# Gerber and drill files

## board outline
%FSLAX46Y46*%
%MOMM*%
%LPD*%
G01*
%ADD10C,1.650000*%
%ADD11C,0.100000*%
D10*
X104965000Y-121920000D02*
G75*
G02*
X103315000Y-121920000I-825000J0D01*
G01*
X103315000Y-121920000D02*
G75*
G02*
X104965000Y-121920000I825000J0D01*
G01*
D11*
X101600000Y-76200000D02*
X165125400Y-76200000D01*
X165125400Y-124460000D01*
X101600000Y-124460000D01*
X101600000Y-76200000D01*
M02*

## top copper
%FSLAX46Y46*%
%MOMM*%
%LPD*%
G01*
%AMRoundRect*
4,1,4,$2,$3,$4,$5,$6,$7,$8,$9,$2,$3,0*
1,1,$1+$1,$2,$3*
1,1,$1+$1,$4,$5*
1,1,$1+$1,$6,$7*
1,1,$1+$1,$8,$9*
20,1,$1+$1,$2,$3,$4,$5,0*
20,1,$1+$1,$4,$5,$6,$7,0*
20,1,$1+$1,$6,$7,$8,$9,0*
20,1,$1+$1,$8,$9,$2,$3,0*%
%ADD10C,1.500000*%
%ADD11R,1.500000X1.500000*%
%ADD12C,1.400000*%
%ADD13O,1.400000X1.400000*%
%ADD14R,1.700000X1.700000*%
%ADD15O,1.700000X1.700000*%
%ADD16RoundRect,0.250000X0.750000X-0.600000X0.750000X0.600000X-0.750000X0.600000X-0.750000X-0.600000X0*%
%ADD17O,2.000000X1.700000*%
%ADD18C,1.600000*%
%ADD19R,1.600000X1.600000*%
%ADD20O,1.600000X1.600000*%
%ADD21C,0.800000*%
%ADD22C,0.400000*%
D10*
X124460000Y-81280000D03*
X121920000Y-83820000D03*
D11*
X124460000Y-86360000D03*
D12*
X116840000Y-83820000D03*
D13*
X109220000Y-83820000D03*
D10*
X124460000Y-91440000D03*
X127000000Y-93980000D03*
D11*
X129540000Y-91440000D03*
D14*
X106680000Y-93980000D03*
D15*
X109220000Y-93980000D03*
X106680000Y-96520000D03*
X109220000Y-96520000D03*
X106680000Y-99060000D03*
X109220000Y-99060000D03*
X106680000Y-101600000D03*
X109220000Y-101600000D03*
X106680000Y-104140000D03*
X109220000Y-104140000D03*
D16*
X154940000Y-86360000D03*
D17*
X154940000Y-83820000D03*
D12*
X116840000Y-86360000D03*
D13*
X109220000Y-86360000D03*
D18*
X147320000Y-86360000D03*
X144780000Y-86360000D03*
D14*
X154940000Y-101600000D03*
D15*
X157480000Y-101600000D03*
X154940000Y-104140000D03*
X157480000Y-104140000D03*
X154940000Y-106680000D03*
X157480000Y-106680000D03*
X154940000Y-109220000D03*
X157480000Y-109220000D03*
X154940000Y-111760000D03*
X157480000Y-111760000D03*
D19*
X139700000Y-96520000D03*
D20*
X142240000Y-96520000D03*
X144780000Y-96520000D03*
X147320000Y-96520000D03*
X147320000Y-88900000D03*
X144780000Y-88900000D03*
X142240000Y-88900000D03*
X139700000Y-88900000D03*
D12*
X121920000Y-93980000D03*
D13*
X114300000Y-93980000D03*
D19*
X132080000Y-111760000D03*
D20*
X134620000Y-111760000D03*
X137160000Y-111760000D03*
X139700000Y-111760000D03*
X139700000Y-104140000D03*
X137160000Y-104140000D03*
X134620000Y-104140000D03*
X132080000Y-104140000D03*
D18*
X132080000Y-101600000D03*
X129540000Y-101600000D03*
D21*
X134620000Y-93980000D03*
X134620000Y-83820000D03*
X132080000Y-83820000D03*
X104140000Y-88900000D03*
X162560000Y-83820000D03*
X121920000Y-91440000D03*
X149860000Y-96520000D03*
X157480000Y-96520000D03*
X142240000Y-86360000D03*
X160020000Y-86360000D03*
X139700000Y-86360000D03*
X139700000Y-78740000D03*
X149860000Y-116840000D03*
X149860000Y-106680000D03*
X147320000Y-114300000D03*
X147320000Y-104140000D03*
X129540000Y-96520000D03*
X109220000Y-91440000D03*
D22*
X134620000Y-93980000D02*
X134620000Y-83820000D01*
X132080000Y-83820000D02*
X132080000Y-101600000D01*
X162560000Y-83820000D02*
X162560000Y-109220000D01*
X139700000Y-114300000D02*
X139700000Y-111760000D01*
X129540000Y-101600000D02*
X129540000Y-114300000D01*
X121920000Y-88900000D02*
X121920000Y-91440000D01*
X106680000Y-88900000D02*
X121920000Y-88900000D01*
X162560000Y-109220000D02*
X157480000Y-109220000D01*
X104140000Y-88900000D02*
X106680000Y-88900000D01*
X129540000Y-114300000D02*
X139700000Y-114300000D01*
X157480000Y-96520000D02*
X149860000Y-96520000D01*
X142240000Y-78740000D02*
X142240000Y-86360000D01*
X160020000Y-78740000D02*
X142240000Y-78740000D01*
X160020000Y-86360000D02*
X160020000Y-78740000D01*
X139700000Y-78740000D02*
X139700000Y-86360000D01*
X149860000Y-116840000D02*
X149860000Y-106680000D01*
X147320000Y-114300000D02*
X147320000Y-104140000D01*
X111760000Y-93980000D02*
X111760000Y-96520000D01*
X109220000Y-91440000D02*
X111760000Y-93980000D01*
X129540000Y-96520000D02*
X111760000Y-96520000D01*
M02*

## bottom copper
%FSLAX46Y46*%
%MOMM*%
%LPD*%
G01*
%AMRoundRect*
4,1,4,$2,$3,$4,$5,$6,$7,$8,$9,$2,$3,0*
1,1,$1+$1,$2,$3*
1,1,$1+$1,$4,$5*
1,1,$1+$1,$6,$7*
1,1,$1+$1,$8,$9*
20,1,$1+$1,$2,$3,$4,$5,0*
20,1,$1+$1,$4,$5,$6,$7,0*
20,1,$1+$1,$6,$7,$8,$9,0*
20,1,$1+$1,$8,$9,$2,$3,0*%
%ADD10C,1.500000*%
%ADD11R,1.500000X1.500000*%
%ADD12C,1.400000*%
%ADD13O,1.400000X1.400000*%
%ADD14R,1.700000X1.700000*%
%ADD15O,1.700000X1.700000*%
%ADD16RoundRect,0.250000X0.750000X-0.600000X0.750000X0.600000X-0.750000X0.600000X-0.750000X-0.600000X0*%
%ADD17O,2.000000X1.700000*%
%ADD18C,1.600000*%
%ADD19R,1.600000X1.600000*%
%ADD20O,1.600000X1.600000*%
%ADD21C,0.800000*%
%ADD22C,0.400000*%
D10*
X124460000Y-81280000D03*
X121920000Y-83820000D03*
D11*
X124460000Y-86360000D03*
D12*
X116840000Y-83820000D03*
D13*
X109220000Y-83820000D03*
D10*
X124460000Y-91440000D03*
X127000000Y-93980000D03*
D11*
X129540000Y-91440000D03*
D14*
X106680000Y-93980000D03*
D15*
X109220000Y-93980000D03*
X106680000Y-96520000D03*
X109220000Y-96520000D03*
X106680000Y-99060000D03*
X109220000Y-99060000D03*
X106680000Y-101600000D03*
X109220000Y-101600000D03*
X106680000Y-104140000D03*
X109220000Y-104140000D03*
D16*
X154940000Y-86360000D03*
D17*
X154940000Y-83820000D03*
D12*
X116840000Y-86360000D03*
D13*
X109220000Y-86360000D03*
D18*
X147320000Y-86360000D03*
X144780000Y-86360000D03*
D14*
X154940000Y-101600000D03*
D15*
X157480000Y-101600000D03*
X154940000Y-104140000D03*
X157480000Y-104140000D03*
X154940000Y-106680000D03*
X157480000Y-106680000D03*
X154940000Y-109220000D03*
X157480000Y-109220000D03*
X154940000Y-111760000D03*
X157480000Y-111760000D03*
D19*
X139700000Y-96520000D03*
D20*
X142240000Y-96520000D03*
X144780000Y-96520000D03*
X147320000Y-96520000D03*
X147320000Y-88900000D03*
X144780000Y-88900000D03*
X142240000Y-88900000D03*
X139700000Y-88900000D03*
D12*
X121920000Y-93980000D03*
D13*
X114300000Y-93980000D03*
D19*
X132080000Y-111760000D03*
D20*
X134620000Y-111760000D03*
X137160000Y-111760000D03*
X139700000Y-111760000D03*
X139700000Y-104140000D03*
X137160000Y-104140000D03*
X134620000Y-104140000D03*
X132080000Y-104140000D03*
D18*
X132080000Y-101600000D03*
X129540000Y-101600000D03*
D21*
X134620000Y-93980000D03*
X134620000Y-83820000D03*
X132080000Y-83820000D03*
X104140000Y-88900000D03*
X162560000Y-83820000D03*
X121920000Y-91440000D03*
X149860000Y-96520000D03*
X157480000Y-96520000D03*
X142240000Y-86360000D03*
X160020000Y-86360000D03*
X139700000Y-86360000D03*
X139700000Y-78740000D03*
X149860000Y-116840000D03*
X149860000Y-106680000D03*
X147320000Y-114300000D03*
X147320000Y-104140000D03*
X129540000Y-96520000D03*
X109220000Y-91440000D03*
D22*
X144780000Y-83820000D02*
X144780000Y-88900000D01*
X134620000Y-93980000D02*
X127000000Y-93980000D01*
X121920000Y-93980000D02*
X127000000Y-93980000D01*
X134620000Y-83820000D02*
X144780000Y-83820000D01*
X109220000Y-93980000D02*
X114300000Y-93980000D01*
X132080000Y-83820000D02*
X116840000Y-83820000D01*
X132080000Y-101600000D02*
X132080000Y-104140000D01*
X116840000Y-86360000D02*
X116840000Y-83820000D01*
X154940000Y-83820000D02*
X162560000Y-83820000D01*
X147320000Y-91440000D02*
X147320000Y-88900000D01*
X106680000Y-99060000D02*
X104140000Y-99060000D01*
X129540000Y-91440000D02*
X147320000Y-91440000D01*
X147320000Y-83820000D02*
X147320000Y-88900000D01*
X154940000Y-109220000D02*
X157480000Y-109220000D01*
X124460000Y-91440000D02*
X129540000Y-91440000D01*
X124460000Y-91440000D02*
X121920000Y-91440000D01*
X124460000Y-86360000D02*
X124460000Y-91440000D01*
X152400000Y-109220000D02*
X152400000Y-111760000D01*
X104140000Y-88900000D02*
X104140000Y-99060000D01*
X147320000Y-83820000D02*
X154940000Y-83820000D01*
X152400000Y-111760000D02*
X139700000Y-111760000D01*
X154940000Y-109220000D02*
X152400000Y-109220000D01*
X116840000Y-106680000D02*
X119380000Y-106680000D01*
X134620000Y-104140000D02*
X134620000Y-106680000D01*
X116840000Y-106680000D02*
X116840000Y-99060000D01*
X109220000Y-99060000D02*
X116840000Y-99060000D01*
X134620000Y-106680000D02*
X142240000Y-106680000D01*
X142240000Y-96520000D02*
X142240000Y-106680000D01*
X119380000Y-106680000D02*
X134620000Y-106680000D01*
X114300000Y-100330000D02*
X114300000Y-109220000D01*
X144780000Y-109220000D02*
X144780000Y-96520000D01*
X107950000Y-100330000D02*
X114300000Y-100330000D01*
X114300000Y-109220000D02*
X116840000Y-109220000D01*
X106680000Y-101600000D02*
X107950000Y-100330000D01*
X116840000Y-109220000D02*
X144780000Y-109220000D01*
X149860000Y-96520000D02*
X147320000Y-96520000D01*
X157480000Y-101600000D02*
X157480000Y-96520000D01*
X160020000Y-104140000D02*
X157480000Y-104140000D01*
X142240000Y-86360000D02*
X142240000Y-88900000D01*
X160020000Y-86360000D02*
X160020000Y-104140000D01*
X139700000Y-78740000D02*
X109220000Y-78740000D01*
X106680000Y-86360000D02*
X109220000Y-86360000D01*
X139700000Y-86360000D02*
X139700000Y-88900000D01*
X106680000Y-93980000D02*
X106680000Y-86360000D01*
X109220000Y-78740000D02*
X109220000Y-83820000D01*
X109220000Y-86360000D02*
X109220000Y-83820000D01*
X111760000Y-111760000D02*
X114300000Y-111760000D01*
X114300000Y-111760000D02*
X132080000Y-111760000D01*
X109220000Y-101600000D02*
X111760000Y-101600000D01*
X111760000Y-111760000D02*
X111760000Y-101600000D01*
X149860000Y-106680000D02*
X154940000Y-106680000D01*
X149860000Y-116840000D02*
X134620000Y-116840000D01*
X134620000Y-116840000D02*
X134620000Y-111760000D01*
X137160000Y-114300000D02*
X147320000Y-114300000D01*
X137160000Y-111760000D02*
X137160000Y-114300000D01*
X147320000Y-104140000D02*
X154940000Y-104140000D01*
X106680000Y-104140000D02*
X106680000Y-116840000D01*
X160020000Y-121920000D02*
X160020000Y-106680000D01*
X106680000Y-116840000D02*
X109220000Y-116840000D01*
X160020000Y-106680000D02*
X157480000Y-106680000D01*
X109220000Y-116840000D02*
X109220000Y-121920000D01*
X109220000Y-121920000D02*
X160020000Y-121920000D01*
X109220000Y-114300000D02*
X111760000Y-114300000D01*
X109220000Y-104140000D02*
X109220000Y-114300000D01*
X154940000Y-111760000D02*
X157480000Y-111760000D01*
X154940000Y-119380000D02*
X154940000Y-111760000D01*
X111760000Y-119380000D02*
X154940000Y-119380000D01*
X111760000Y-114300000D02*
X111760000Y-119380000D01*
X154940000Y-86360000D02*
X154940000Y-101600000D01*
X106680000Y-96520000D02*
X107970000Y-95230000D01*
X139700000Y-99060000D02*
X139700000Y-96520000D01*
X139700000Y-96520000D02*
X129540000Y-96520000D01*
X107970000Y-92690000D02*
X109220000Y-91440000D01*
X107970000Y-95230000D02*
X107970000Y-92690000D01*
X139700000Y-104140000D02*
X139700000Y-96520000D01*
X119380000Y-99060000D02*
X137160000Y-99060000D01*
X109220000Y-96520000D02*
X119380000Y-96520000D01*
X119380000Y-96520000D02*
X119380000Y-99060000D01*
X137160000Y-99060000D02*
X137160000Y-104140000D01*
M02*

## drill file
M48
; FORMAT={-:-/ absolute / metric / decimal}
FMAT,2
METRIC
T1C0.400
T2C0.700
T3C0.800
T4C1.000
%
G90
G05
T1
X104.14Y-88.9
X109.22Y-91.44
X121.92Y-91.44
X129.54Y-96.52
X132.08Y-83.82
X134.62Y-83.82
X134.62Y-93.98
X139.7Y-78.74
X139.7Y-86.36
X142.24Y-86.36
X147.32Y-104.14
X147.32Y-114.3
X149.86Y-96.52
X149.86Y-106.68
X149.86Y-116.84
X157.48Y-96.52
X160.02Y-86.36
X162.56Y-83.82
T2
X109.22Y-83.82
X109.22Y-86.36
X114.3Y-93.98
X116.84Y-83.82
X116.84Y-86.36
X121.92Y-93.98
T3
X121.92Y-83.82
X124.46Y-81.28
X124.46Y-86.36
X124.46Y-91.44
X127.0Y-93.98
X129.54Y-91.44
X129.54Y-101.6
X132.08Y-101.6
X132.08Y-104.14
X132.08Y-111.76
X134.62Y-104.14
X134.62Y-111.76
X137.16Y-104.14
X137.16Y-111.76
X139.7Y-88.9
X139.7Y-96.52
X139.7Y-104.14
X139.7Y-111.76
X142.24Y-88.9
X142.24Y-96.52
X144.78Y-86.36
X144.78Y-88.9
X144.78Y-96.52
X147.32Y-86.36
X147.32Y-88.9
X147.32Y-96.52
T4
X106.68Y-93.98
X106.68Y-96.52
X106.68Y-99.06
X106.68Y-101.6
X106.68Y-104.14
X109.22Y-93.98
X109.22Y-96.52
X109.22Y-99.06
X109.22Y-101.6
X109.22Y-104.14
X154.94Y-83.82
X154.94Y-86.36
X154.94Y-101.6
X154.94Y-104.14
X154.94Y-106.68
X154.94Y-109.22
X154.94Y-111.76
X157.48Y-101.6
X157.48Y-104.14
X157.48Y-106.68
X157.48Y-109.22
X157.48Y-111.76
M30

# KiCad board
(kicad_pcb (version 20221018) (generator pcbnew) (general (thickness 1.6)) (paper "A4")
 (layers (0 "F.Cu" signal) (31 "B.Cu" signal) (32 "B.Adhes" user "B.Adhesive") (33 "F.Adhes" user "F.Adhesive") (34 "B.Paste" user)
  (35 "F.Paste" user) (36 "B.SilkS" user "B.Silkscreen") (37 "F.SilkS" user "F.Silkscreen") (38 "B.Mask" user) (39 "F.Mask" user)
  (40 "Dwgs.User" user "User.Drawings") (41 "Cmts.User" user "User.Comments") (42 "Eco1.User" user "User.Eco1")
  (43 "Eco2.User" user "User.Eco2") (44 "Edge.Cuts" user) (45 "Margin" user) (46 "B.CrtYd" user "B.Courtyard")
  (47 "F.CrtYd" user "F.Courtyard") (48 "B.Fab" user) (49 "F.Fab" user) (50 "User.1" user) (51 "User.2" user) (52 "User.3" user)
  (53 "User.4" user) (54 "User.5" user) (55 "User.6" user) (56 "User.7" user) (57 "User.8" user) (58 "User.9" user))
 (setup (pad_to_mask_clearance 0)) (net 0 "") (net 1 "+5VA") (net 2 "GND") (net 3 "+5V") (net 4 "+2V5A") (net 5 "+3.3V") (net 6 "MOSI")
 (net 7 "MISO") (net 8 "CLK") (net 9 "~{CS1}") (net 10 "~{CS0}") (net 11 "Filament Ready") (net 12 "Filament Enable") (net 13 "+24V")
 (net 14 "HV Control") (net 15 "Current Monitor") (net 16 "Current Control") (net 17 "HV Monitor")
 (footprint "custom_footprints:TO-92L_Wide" (layer "F.Cu") (at 124.46 86.36 90)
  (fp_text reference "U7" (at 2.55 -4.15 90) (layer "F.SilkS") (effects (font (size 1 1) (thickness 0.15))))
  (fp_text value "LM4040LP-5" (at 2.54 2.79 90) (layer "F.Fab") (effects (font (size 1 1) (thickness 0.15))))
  (pad "1" thru_hole circle (at 5.08 0 90) (size 1.5 1.5) (drill 0.8) (layers "*.Cu" "*.Mask"))
  (pad "2" thru_hole circle (at 2.54 -2.54 90) (size 1.5 1.5) (drill 0.8) (layers "*.Cu" "*.Mask") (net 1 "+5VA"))
  (pad "3" thru_hole rect (at 0 0 90) (size 1.5 1.5) (drill 0.8) (layers "*.Cu" "*.Mask") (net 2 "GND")))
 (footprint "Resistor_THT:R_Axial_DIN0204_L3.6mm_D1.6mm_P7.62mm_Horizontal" (layer "F.Cu") (at 116.84 83.82 180)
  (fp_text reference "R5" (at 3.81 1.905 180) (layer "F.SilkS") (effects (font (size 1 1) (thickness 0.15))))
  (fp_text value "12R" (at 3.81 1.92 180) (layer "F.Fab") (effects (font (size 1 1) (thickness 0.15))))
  (pad "1" thru_hole circle (at 0 0 180) (size 1.4 1.4) (drill 0.7) (layers "*.Cu" "*.Mask") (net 1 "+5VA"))
  (pad "2" thru_hole oval (at 7.62 0 180) (size 1.4 1.4) (drill 0.7) (layers "*.Cu" "*.Mask") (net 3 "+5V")))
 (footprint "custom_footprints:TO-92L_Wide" (layer "F.Cu") (at 129.54 91.44 180)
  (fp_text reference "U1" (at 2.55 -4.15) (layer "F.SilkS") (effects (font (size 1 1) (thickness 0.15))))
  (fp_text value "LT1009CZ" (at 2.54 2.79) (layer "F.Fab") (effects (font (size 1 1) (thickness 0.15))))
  (pad "1" thru_hole circle (at 5.08 0 180) (size 1.5 1.5) (drill 0.8) (layers "*.Cu" "*.Mask") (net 2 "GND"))
  (pad "2" thru_hole circle (at 2.54 -2.54 180) (size 1.5 1.5) (drill 0.8) (layers "*.Cu" "*.Mask") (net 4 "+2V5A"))
  (pad "3" thru_hole rect (at 0 0 180) (size 1.5 1.5) (drill 0.8) (layers "*.Cu" "*.Mask") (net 2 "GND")))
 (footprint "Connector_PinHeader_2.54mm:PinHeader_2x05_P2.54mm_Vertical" (layer "F.Cu") (at 106.68 93.98)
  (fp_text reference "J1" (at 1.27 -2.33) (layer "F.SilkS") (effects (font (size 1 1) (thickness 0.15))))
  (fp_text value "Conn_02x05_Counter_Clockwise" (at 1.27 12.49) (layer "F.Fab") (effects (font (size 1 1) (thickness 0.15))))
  (pad "1" thru_hole rect (at 0 0) (size 1.7 1.7) (drill 1) (layers "*.Cu" "*.Mask") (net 3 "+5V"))
  (pad "2" thru_hole oval (at 2.54 0) (size 1.7 1.7) (drill 1) (layers "*.Cu" "*.Mask") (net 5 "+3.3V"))
  (pad "3" thru_hole oval (at 0 2.54) (size 1.7 1.7) (drill 1) (layers "*.Cu" "*.Mask") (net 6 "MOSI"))
  (pad "4" thru_hole oval (at 2.54 2.54) (size 1.7 1.7) (drill 1) (layers "*.Cu" "*.Mask") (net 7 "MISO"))
  (pad "5" thru_hole oval (at 0 5.08) (size 1.7 1.7) (drill 1) (layers "*.Cu" "*.Mask") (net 2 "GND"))
  (pad "6" thru_hole oval (at 2.54 5.08) (size 1.7 1.7) (drill 1) (layers "*.Cu" "*.Mask") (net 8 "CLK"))
  (pad "7" thru_hole oval (at 0 7.62) (size 1.7 1.7) (drill 1) (layers "*.Cu" "*.Mask") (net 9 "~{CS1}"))
  (pad "8" thru_hole oval (at 2.54 7.62) (size 1.7 1.7) (drill 1) (layers "*.Cu" "*.Mask") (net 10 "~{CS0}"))
  (pad "9" thru_hole oval (at 0 10.16) (size 1.7 1.7) (drill 1) (layers "*.Cu" "*.Mask") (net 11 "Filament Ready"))
  (pad "10" thru_hole oval (at 2.54 10.16) (size 1.7 1.7) (drill 1) (layers "*.Cu" "*.Mask") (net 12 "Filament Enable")))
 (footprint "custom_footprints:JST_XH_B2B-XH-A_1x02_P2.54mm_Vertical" (layer "F.Cu") (at 154.94 86.34 90)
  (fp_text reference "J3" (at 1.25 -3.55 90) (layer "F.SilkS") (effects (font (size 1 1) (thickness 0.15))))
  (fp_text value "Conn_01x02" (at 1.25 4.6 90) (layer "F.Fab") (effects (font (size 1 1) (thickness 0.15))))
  (pad "1" thru_hole roundrect (at -0.02 0 90) (size 1.7 2) (drill 1) (layers "*.Cu" "*.Mask") (roundrect_rratio 0.1470588235)
   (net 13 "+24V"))
  (pad "2" thru_hole oval (at 2.52 0 90) (size 1.7 2) (drill 1) (layers "*.Cu" "*.Mask") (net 2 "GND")))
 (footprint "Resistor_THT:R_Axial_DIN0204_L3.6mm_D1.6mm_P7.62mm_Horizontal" (layer "F.Cu") (at 116.84 86.36 180)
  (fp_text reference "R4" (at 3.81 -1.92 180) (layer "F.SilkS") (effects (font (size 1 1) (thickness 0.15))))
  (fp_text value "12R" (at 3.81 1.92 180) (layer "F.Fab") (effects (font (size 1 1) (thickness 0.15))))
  (pad "1" thru_hole circle (at 0 0 180) (size 1.4 1.4) (drill 0.7) (layers "*.Cu" "*.Mask") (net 1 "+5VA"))
  (pad "2" thru_hole oval (at 7.62 0 180) (size 1.4 1.4) (drill 0.7) (layers "*.Cu" "*.Mask") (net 3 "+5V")))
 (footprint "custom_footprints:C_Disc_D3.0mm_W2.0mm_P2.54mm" (layer "F.Cu") (at 147.3 86.36 180)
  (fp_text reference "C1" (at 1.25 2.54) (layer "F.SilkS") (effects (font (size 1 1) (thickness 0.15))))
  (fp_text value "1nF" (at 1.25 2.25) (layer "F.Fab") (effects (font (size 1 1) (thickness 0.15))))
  (pad "1" thru_hole circle (at -0.02 0 180) (size 1.6 1.6) (drill 0.8) (layers "*.Cu" "*.Mask") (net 2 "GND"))
  (pad "2" thru_hole circle (at 2.52 0 180) (size 1.6 1.6) (drill 0.8) (layers "*.Cu" "*.Mask") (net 4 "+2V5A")))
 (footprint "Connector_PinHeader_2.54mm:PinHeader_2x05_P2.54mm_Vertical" (layer "F.Cu") (at 154.94 101.6)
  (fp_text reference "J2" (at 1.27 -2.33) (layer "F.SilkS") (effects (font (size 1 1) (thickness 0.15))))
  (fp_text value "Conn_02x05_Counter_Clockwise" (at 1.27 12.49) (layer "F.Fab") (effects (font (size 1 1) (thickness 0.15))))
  (pad "1" thru_hole rect (at 0 0) (size 1.7 1.7) (drill 1) (layers "*.Cu" "*.Mask") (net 13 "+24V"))
  (pad "2" thru_hole oval (at 2.54 0) (size 1.7 1.7) (drill 1) (layers "*.Cu" "*.Mask") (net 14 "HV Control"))
  (pad "3" thru_hole oval (at 0 2.54) (size 1.7 1.7) (drill 1) (layers "*.Cu" "*.Mask") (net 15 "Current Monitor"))
  (pad "4" thru_hole oval (at 2.54 2.54) (size 1.7 1.7) (drill 1) (layers "*.Cu" "*.Mask") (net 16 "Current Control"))
  (pad "5" thru_hole oval (at 0 5.08) (size 1.7 1.7) (drill 1) (layers "*.Cu" "*.Mask") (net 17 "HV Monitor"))
  (pad "6" thru_hole oval (at 2.54 5.08) (size 1.7 1.7) (drill 1) (layers "*.Cu" "*.Mask") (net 11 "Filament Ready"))
  (pad "7" thru_hole oval (at 0 7.62) (size 1.7 1.7) (drill 1) (layers "*.Cu" "*.Mask") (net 2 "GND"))
  (pad "8" thru_hole oval (at 2.54 7.62) (size 1.7 1.7) (drill 1) (layers "*.Cu" "*.Mask") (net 2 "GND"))
  (pad "9" thru_hole oval (at 0 10.16) (size 1.7 1.7) (drill 1) (layers "*.Cu" "*.Mask") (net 12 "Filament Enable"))
  (pad "10" thru_hole oval (at 2.54 10.16) (size 1.7 1.7) (drill 1) (layers "*.Cu" "*.Mask") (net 12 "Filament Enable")))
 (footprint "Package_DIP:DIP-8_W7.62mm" (layer "F.Cu") (at 139.7 96.52 90)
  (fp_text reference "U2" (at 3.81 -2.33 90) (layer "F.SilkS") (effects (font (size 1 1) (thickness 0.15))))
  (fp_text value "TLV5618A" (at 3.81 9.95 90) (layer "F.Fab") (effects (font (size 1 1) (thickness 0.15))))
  (pad "1" thru_hole rect (at 0 0 90) (size 1.6 1.6) (drill 0.8) (layers "*.Cu" "*.Mask") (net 6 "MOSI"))
  (pad "2" thru_hole oval (at 0 2.54 90) (size 1.6 1.6) (drill 0.8) (layers "*.Cu" "*.Mask") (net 8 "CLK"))
  (pad "3" thru_hole oval (at 0 5.08 90) (size 1.6 1.6) (drill 0.8) (layers "*.Cu" "*.Mask") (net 9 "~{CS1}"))
  (pad "4" thru_hole oval (at 0 7.62 90) (size 1.6 1.6) (drill 0.8) (layers "*.Cu" "*.Mask") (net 14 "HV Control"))
  (pad "5" thru_hole oval (at 7.62 7.62 90) (size 1.6 1.6) (drill 0.8) (layers "*.Cu" "*.Mask") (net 2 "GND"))
  (pad "6" thru_hole oval (at 7.62 5.08 90) (size 1.6 1.6) (drill 0.8) (layers "*.Cu" "*.Mask") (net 4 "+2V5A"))
  (pad "7" thru_hole oval (at 7.62 2.54 90) (size 1.6 1.6) (drill 0.8) (layers "*.Cu" "*.Mask") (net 16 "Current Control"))
  (pad "8" thru_hole oval (at 7.62 0 90) (size 1.6 1.6) (drill 0.8) (layers "*.Cu" "*.Mask") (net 3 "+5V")))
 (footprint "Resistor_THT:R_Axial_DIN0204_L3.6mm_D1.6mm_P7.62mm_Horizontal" (layer "F.Cu") (at 121.92 93.98 180)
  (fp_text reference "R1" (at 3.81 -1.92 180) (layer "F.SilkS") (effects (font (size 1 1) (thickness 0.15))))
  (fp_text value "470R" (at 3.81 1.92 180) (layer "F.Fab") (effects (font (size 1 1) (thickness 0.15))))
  (pad "1" thru_hole circle (at 0 0 180) (size 1.4 1.4) (drill 0.7) (layers "*.Cu" "*.Mask") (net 4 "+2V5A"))
  (pad "2" thru_hole oval (at 7.62 0 180) (size 1.4 1.4) (drill 0.7) (layers "*.Cu" "*.Mask") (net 5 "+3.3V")))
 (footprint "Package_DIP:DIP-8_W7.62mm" (layer "F.Cu") (at 132.08 111.76 90)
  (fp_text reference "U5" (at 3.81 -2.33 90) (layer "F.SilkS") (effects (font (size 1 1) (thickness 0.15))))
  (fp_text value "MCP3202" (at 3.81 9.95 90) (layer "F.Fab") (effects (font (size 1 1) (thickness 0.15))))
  (pad "1" thru_hole rect (at 0 0 90) (size 1.6 1.6) (drill 0.8) (layers "*.Cu" "*.Mask") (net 10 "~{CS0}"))
  (pad "2" thru_hole oval (at 0 2.54 90) (size 1.6 1.6) (drill 0.8) (layers "*.Cu" "*.Mask") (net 17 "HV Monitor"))
  (pad "3" thru_hole oval (at 0 5.08 90) (size 1.6 1.6) (drill 0.8) (layers "*.Cu" "*.Mask") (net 15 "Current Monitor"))
  (pad "4" thru_hole oval (at 0 7.62 90) (size 1.6 1.6) (drill 0.8) (layers "*.Cu" "*.Mask") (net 2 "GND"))
  (pad "5" thru_hole oval (at 7.62 7.62 90) (size 1.6 1.6) (drill 0.8) (layers "*.Cu" "*.Mask") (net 6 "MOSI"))
  (pad "6" thru_hole oval (at 7.62 5.08 90) (size 1.6 1.6) (drill 0.8) (layers "*.Cu" "*.Mask") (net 7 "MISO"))
  (pad "7" thru_hole oval (at 7.62 2.54 90) (size 1.6 1.6) (drill 0.8) (layers "*.Cu" "*.Mask") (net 8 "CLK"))
  (pad "8" thru_hole oval (at 7.62 0 90) (size 1.6 1.6) (drill 0.8) (layers "*.Cu" "*.Mask") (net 1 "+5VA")))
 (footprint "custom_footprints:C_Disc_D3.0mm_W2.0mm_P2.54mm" (layer "F.Cu") (at 132.06 101.6 180)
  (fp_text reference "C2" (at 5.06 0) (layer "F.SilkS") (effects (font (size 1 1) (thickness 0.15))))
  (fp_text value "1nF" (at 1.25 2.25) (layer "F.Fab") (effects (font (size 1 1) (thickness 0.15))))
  (pad "1" thru_hole circle (at -0.02 0 180) (size 1.6 1.6) (drill 0.8) (layers "*.Cu" "*.Mask") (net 1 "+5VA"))
  (pad "2" thru_hole circle (at 2.52 0 180) (size 1.6 1.6) (drill 0.8) (layers "*.Cu" "*.Mask") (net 2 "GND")))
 (gr_circle (center 104.14 121.92) (end 105.74 121.92) (stroke (width 0.1) (type solid)) (fill solid) (layer "Edge.Cuts"))
 (gr_rect (start 101.6 76.2) (end 165.1254 124.46) (stroke (width 0.1) (type default)) (fill none) (layer "Edge.Cuts"))
 (segment (start 134.62 93.98) (end 134.62 83.82) (width 0.4) (layer "F.Cu") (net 4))
 (via (at 134.62 93.98) (size 0.8) (drill 0.4) (layers "F.Cu" "B.Cu") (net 4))
 (via (at 134.62 83.82) (size 0.8) (drill 0.4) (layers "F.Cu" "B.Cu") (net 4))
 (segment (start 144.78 83.82) (end 144.78 88.9) (width 0.4) (layer "B.Cu") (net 4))
 (segment (start 134.62 93.98) (end 127 93.98) (width 0.4) (layer "B.Cu") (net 4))
 (segment (start 121.92 93.98) (end 127 93.98) (width 0.4) (layer "B.Cu") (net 4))
 (segment (start 134.62 83.82) (end 144.78 83.82) (width 0.4) (layer "B.Cu") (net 4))
 (segment (start 109.22 93.98) (end 114.3 93.98) (width 0.4) (layer "B.Cu") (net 5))
 (segment (start 132.08 83.82) (end 132.08 101.6) (width 0.4) (layer "F.Cu") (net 1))
 (via (at 132.08 83.82) (size 0.8) (drill 0.4) (layers "F.Cu" "B.Cu") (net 1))
 (segment (start 132.08 83.82) (end 116.84 83.82) (width 0.4) (layer "B.Cu") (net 1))
 (segment (start 132.08 101.6) (end 132.08 104.14) (width 0.4) (layer "B.Cu") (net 1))
 (segment (start 116.84 86.36) (end 116.84 83.82) (width 0.4) (layer "B.Cu") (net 1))
 (segment (start 162.56 83.82) (end 162.56 109.22) (width 0.4) (layer "F.Cu") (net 2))
 (segment (start 139.7 114.3) (end 139.7 111.76) (width 0.4) (layer "F.Cu") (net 2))
 (segment (start 129.54 101.6) (end 129.54 114.3) (width 0.4) (layer "F.Cu") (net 2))
 (segment (start 121.92 88.9) (end 121.92 91.44) (width 0.4) (layer "F.Cu") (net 2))
 (segment (start 106.68 88.9) (end 121.92 88.9) (width 0.4) (layer "F.Cu") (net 2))
 (segment (start 162.56 109.22) (end 157.48 109.22) (width 0.4) (layer "F.Cu") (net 2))
 (segment (start 104.14 88.9) (end 106.68 88.9) (width 0.4) (layer "F.Cu") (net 2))
 (segment (start 129.54 114.3) (end 139.7 114.3) (width 0.4) (layer "F.Cu") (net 2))
 (via (at 104.14 88.9) (size 0.8) (drill 0.4) (layers "F.Cu" "B.Cu") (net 2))
 (via (at 162.56 83.82) (size 0.8) (drill 0.4) (layers "F.Cu" "B.Cu") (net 2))
 (via (at 121.92 91.44) (size 0.8) (drill 0.4) (layers "F.Cu" "B.Cu") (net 2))
 (segment (start 154.94 83.82) (end 162.56 83.82) (width 0.4) (layer "B.Cu") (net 2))
 (segment (start 147.32 91.44) (end 147.32 88.9) (width 0.4) (layer "B.Cu") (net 2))
 (segment (start 106.68 99.06) (end 104.14 99.06) (width 0.4) (layer "B.Cu") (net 2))
 (segment (start 129.54 91.44) (end 147.32 91.44) (width 0.4) (layer "B.Cu") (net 2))
 (segment (start 147.32 83.82) (end 147.32 88.9) (width 0.4) (layer "B.Cu") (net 2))
 (segment (start 154.94 109.22) (end 157.48 109.22) (width 0.4) (layer "B.Cu") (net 2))
 (segment (start 124.46 91.44) (end 129.54 91.44) (width 0.4) (layer "B.Cu") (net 2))
 (segment (start 124.46 91.44) (end 121.92 91.44) (width 0.4) (layer "B.Cu") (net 2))
 (segment (start 124.46 86.36) (end 124.46 91.44) (width 0.4) (layer "B.Cu") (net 2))
 (segment (start 152.4 109.22) (end 152.4 111.76) (width 0.4) (layer "B.Cu") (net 2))
 (segment (start 104.14 88.9) (end 104.14 99.06) (width 0.4) (layer "B.Cu") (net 2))
 (segment (start 147.32 83.82) (end 154.94 83.82) (width 0.4) (layer "B.Cu") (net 2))
 (segment (start 152.4 111.76) (end 139.7 111.76) (width 0.4) (layer "B.Cu") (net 2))
 (segment (start 154.94 109.22) (end 152.4 109.22) (width 0.4) (layer "B.Cu") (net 2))
 (segment (start 116.84 106.68) (end 119.38 106.68) (width 0.4) (layer "B.Cu") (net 8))
 (segment (start 134.62 104.14) (end 134.62 106.68) (width 0.4) (layer "B.Cu") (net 8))
 (segment (start 116.84 106.68) (end 116.84 99.06) (width 0.4) (layer "B.Cu") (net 8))
 (segment (start 109.22 99.06) (end 116.84 99.06) (width 0.4) (layer "B.Cu") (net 8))
 (segment (start 134.62 106.68) (end 142.24 106.68) (width 0.4) (layer "B.Cu") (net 8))
 (segment (start 142.24 96.52) (end 142.24 106.68) (width 0.4) (layer "B.Cu") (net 8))
 (segment (start 119.38 106.68) (end 134.62 106.68) (width 0.4) (layer "B.Cu") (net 8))
 (segment (start 114.3 100.33) (end 114.3 109.22) (width 0.4) (layer "B.Cu") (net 9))
 (segment (start 144.78 109.22) (end 144.78 96.52) (width 0.4) (layer "B.Cu") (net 9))
 (segment (start 107.95 100.33) (end 114.3 100.33) (width 0.4) (layer "B.Cu") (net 9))
 (segment (start 114.3 109.22) (end 116.84 109.22) (width 0.4) (layer "B.Cu") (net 9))
 (segment (start 106.68 101.6) (end 107.95 100.33) (width 0.4) (layer "B.Cu") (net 9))
 (segment (start 116.84 109.22) (end 144.78 109.22) (width 0.4) (layer "B.Cu") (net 9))
 (segment (start 157.48 96.52) (end 149.86 96.52) (width 0.4) (layer "F.Cu") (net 14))
 (via (at 149.86 96.52) (size 0.8) (drill 0.4) (layers "F.Cu" "B.Cu") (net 14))
 (via (at 157.48 96.52) (size 0.8) (drill 0.4) (layers "F.Cu" "B.Cu") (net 14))
 (segment (start 149.86 96.52) (end 147.32 96.52) (width 0.4) (layer "B.Cu") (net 14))
 (segment (start 157.48 101.6) (end 157.48 96.52) (width 0.4) (layer "B.Cu") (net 14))
 (segment (start 142.24 78.74) (end 142.24 86.36) (width 0.4) (layer "F.Cu") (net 16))
 (segment (start 160.02 78.74) (end 142.24 78.74) (width 0.4) (layer "F.Cu") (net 16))
 (segment (start 160.02 86.36) (end 160.02 78.74) (width 0.4) (layer "F.Cu") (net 16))
 (via (at 142.24 86.36) (size 0.8) (drill 0.4) (layers "F.Cu" "B.Cu") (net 16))
 (via (at 160.02 86.36) (size 0.8) (drill 0.4) (layers "F.Cu" "B.Cu") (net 16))
 (segment (start 160.02 104.14) (end 157.48 104.14) (width 0.4) (layer "B.Cu") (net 16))
 (segment (start 142.24 86.36) (end 142.24 88.9) (width 0.4) (layer "B.Cu") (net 16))
 (segment (start 160.02 86.36) (end 160.02 104.14) (width 0.4) (layer "B.Cu") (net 16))
 (segment (start 139.7 78.74) (end 139.7 86.36) (width 0.4) (layer "F.Cu") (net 3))
 (via (at 139.7 86.36) (size 0.8) (drill 0.4) (layers "F.Cu" "B.Cu") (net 3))
 (via (at 139.7 78.74) (size 0.8) (drill 0.4) (layers "F.Cu" "B.Cu") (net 3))
 (segment (start 139.7 78.74) (end 109.22 78.74) (width 0.4) (layer "B.Cu") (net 3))
 (segment (start 106.68 86.36) (end 109.22 86.36) (width 0.4) (layer "B.Cu") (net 3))
 (segment (start 139.7 86.36) (end 139.7 88.9) (width 0.4) (layer "B.Cu") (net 3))
 (segment (start 106.68 93.98) (end 106.68 86.36) (width 0.4) (layer "B.Cu") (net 3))
 (segment (start 109.22 78.74) (end 109.22 83.82) (width 0.4) (layer "B.Cu") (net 3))
 (segment (start 109.22 86.36) (end 109.22 83.82) (width 0.4) (layer "B.Cu") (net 3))
 (segment (start 111.76 111.76) (end 114.3 111.76) (width 0.4) (layer "B.Cu") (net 10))
 (segment (start 114.3 111.76) (end 132.08 111.76) (width 0.4) (layer "B.Cu") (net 10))
 (segment (start 109.22 101.6) (end 111.76 101.6) (width 0.4) (layer "B.Cu") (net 10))
 (segment (start 111.76 111.76) (end 111.76 101.6) (width 0.4) (layer "B.Cu") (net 10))
 (segment (start 149.86 116.84) (end 149.86 106.68) (width 0.4) (layer "F.Cu") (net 17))
 (via (at 149.86 116.84) (size 0.8) (drill 0.4) (layers "F.Cu" "B.Cu") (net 17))
 (via (at 149.86 106.68) (size 0.8) (drill 0.4) (layers "F.Cu" "B.Cu") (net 17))
 (segment (start 149.86 106.68) (end 154.94 106.68) (width 0.4) (layer "B.Cu") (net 17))
 (segment (start 149.86 116.84) (end 134.62 116.84) (width 0.4) (layer "B.Cu") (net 17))
 (segment (start 134.62 116.84) (end 134.62 111.76) (width 0.4) (layer "B.Cu") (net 17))
 (segment (start 147.32 114.3) (end 147.32 104.14) (width 0.4) (layer "F.Cu") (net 15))
 (via (at 147.32 114.3) (size 0.8) (drill 0.4) (layers "F.Cu" "B.Cu") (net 15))
 (via (at 147.32 104.14) (size 0.8) (drill 0.4) (layers "F.Cu" "B.Cu") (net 15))
 (segment (start 137.16 114.3) (end 147.32 114.3) (width 0.4) (layer "B.Cu") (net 15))
 (segment (start 137.16 111.76) (end 137.16 114.3) (width 0.4) (layer "B.Cu") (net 15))
 (segment (start 147.32 104.14) (end 154.94 104.14) (width 0.4) (layer "B.Cu") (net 15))
 (segment (start 106.68 104.14) (end 106.68 116.84) (width 0.4) (layer "B.Cu") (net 11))
 (segment (start 160.02 121.92) (end 160.02 106.68) (width 0.4) (layer "B.Cu") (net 11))
 (segment (start 106.68 116.84) (end 109.22 116.84) (width 0.4) (layer "B.Cu") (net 11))
 (segment (start 160.02 106.68) (end 157.48 106.68) (width 0.4) (layer "B.Cu") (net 11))
 (segment (start 109.22 116.84) (end 109.22 121.92) (width 0.4) (layer "B.Cu") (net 11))
 (segment (start 109.22 121.92) (end 160.02 121.92) (width 0.4) (layer "B.Cu") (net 11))
 (segment (start 109.22 114.3) (end 111.76 114.3) (width 0.4) (layer "B.Cu") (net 12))
 (segment (start 109.22 104.14) (end 109.22 114.3) (width 0.4) (layer "B.Cu") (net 12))
 (segment (start 154.94 111.76) (end 157.48 111.76) (width 0.4) (layer "B.Cu") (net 12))
 (segment (start 154.94 119.38) (end 154.94 111.76) (width 0.4) (layer "B.Cu") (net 12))
 (segment (start 111.76 119.38) (end 154.94 119.38) (width 0.4) (layer "B.Cu") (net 12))
 (segment (start 111.76 114.3) (end 111.76 119.38) (width 0.4) (layer "B.Cu") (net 12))
 (segment (start 154.94 86.36) (end 154.94 101.6) (width 0.4) (layer "B.Cu") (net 13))
 (segment (start 111.76 93.98) (end 111.76 96.52) (width 0.4) (layer "F.Cu") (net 6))
 (segment (start 109.22 91.44) (end 111.76 93.98) (width 0.4) (layer "F.Cu") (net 6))
 (segment (start 129.54 96.52) (end 111.76 96.52) (width 0.4) (layer "F.Cu") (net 6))
 (via (at 129.54 96.52) (size 0.8) (drill 0.4) (layers "F.Cu" "B.Cu") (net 6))
 (via (at 109.22 91.44) (size 0.8) (drill 0.4) (layers "F.Cu" "B.Cu") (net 6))
 (segment (start 106.68 96.52) (end 107.97 95.23) (width 0.4) (layer "B.Cu") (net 6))
 (segment (start 139.7 99.06) (end 139.7 96.52) (width 0.4) (layer "B.Cu") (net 6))
 (segment (start 139.7 96.52) (end 129.54 96.52) (width 0.4) (layer "B.Cu") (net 6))
 (segment (start 107.97 92.69) (end 109.22 91.44) (width 0.4) (layer "B.Cu") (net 6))
 (segment (start 107.97 95.23) (end 107.97 92.69) (width 0.4) (layer "B.Cu") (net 6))
 (segment (start 139.7 104.14) (end 139.7 96.52) (width 0.4) (layer "B.Cu") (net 6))
 (segment (start 119.38 99.06) (end 137.16 99.06) (width 0.4) (layer "B.Cu") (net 7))
 (segment (start 109.22 96.52) (end 119.38 96.52) (width 0.4) (layer "B.Cu") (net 7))
 (segment (start 119.38 96.52) (end 119.38 99.06) (width 0.4) (layer "B.Cu") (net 7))
 (segment (start 137.16 99.06) (end 137.16 104.14) (width 0.4) (layer "B.Cu") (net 7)))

